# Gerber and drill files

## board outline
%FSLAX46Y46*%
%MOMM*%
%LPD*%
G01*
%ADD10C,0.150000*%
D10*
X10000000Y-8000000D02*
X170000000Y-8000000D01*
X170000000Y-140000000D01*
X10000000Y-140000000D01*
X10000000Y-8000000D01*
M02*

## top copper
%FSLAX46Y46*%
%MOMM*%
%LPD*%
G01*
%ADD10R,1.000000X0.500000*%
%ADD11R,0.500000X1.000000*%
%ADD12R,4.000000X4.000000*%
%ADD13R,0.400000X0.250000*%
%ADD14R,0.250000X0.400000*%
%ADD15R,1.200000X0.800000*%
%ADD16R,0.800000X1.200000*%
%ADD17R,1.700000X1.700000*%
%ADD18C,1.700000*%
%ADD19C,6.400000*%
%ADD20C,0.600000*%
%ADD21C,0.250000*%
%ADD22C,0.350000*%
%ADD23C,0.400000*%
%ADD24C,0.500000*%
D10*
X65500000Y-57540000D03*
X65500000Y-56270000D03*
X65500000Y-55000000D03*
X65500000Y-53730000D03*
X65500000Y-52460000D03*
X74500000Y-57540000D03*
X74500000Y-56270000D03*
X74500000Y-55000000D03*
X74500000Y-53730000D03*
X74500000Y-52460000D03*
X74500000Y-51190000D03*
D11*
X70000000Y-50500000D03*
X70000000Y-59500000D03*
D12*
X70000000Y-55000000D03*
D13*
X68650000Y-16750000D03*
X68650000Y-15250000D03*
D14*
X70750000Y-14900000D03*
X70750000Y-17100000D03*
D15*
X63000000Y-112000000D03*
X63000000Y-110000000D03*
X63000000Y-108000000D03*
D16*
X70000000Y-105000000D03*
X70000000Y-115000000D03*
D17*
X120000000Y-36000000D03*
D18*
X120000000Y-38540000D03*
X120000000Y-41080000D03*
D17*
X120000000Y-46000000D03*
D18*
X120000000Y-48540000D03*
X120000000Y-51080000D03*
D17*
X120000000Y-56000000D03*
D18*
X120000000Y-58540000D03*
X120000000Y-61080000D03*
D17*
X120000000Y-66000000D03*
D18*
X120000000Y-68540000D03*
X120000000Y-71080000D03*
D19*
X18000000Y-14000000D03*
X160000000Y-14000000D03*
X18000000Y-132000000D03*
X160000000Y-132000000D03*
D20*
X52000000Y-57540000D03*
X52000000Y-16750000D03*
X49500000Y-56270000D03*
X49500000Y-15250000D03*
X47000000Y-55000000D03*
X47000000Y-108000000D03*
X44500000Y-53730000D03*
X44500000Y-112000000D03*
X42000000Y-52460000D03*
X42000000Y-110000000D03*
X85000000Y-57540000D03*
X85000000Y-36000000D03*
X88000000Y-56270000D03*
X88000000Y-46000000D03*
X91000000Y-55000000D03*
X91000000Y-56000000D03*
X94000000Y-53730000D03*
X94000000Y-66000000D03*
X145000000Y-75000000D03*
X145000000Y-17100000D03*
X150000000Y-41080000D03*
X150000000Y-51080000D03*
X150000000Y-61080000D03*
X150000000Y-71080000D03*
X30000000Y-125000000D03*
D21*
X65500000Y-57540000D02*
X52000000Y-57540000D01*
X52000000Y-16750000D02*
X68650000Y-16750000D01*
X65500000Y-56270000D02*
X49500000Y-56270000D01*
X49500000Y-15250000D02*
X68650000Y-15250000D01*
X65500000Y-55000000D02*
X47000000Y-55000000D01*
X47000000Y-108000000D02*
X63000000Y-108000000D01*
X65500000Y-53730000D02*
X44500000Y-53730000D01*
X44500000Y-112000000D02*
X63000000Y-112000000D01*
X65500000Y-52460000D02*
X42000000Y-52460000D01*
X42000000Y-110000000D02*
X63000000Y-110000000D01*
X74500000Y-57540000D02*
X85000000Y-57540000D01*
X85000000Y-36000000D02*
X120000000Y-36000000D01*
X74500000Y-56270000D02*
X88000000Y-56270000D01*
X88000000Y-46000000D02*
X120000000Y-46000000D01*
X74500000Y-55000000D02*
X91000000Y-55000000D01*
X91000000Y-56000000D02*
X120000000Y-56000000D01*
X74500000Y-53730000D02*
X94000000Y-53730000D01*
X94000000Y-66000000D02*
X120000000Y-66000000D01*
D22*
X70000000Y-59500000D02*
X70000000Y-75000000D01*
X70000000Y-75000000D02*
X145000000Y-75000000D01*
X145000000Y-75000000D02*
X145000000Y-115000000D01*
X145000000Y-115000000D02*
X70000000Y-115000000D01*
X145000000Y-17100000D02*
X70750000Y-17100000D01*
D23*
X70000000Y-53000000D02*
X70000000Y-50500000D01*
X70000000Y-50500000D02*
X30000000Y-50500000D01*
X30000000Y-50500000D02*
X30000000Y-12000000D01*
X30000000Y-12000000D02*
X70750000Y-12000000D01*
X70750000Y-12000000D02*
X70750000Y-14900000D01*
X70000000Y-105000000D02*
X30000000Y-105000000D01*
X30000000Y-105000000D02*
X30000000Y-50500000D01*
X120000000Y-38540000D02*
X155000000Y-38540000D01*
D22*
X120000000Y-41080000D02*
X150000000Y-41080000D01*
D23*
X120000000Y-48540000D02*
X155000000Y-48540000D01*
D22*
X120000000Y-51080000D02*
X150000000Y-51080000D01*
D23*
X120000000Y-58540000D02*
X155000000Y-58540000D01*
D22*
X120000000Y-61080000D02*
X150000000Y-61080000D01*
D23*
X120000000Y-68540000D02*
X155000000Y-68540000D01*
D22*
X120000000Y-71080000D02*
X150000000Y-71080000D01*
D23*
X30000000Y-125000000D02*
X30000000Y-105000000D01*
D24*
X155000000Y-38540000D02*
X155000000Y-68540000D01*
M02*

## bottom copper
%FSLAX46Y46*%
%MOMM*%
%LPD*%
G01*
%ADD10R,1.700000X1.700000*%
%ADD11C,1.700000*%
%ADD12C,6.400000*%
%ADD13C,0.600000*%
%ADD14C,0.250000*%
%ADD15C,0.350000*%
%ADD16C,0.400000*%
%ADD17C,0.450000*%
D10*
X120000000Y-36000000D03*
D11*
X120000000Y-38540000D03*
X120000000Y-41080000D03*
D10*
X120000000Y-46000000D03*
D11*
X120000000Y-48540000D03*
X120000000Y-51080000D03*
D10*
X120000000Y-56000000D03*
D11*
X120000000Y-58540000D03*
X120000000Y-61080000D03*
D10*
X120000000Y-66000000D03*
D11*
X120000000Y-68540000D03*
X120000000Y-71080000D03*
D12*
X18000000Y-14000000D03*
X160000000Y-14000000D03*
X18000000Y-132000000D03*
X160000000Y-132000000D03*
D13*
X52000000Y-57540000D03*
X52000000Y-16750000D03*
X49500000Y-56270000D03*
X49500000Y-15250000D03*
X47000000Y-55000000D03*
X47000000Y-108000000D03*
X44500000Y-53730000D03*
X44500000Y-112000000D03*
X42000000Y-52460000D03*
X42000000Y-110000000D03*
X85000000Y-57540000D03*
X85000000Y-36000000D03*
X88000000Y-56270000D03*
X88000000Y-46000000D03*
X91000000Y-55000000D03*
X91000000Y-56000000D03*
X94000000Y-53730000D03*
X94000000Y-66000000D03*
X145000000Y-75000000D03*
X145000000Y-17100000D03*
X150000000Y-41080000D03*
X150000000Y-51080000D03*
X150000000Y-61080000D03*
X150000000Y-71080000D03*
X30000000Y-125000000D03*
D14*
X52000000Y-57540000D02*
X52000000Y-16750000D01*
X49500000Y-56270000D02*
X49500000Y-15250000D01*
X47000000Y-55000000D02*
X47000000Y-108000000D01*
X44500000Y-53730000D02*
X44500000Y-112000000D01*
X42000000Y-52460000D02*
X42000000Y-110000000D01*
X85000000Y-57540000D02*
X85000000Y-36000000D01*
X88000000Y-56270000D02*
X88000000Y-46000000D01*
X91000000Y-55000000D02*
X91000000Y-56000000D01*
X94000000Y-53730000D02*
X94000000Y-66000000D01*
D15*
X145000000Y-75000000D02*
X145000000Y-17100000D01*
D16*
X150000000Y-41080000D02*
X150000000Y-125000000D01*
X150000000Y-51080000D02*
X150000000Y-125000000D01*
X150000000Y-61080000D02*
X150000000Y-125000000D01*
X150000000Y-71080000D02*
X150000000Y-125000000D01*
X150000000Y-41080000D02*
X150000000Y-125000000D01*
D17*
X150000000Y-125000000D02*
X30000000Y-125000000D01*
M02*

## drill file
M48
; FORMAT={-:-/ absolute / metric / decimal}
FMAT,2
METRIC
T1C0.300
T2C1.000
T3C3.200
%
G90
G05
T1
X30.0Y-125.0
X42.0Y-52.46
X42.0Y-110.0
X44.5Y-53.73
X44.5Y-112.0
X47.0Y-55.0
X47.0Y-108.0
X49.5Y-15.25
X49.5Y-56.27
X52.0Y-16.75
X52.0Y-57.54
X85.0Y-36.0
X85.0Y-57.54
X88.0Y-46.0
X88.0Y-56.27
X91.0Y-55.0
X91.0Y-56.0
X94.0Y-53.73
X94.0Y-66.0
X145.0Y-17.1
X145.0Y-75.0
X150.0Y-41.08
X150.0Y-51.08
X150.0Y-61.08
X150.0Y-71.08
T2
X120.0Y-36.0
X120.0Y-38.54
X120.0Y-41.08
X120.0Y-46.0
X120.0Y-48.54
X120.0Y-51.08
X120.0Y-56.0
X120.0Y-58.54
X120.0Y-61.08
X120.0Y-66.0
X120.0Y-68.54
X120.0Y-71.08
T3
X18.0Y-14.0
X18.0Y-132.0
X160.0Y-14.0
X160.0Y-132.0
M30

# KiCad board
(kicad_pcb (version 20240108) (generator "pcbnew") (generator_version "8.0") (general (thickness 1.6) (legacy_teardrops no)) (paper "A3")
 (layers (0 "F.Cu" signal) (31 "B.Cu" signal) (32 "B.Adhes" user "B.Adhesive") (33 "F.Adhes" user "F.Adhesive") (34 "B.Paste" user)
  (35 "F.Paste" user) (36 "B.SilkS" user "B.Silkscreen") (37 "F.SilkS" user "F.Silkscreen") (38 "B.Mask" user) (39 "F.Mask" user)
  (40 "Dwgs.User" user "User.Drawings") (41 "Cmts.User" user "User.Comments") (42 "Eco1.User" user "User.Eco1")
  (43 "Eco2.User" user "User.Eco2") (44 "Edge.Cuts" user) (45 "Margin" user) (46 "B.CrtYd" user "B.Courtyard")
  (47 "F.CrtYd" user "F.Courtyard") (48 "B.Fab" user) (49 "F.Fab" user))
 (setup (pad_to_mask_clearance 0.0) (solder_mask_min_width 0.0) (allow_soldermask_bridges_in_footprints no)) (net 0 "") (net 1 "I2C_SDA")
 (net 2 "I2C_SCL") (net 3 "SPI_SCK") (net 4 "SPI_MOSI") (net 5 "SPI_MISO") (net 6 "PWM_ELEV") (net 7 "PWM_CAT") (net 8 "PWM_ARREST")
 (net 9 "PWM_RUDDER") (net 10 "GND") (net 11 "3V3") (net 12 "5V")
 (gr_rect (start 10 8) (end 170 140) (stroke (width 0.15) (type solid)) (fill none) (layer "Edge.Cuts"))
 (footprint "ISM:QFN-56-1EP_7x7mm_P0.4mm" (layer "F.Cu") (at 70 55)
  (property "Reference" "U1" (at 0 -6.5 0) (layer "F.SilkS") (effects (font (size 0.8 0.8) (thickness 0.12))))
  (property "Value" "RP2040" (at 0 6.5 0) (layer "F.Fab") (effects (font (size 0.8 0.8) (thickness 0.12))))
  (pad "1" smd rect (at -4.5 2.54) (size 1.0 0.5) (layers "F.Cu" "F.Paste" "F.Mask") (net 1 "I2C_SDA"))
  (pad "2" smd rect (at -4.5 1.27) (size 1.0 0.5) (layers "F.Cu" "F.Paste" "F.Mask") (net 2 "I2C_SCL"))
  (pad "3" smd rect (at -4.5 0) (size 1.0 0.5) (layers "F.Cu" "F.Paste" "F.Mask") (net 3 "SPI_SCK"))
  (pad "4" smd rect (at -4.5 -1.27) (size 1.0 0.5) (layers "F.Cu" "F.Paste" "F.Mask") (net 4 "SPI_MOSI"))
  (pad "5" smd rect (at -4.5 -2.54) (size 1.0 0.5) (layers "F.Cu" "F.Paste" "F.Mask") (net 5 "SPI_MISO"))
  (pad "6" smd rect (at 4.5 2.54) (size 1.0 0.5) (layers "F.Cu" "F.Paste" "F.Mask") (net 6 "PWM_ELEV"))
  (pad "7" smd rect (at 4.5 1.27) (size 1.0 0.5) (layers "F.Cu" "F.Paste" "F.Mask") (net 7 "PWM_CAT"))
  (pad "8" smd rect (at 4.5 0) (size 1.0 0.5) (layers "F.Cu" "F.Paste" "F.Mask") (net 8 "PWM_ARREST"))
  (pad "9" smd rect (at 4.5 -1.27) (size 1.0 0.5) (layers "F.Cu" "F.Paste" "F.Mask") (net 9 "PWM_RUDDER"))
  (pad "12" smd rect (at 4.5 -2.54) (size 1.0 0.5) (layers "F.Cu" "F.Paste" "F.Mask"))
  (pad "13" smd rect (at 4.5 -3.81) (size 1.0 0.5) (layers "F.Cu" "F.Paste" "F.Mask"))
  (pad "10" smd rect (at 0 -4.5) (size 0.5 1.0) (layers "F.Cu" "F.Paste" "F.Mask") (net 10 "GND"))
  (pad "11" smd rect (at 0 4.5) (size 0.5 1.0) (layers "F.Cu" "F.Paste" "F.Mask") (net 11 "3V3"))
  (pad "EP" smd rect (at 0 0) (size 4 4) (layers "F.Cu" "F.Paste" "F.Mask") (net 10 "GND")))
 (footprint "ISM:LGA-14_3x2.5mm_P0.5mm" (layer "F.Cu") (at 70 16)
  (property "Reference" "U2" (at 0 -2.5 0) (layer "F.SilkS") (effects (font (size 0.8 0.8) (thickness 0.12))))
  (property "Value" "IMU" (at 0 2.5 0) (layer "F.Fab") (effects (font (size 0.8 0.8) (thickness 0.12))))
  (pad "1" smd rect (at -1.35 0.75) (size 0.4 0.25) (layers "F.Cu" "F.Paste" "F.Mask") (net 1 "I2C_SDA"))
  (pad "2" smd rect (at -1.35 -0.75) (size 0.4 0.25) (layers "F.Cu" "F.Paste" "F.Mask") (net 2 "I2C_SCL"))
  (pad "3" smd rect (at 0.75 -1.1) (size 0.25 0.4) (layers "F.Cu" "F.Paste" "F.Mask") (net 10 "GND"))
  (pad "4" smd rect (at 0.75 1.1) (size 0.25 0.4) (layers "F.Cu" "F.Paste" "F.Mask") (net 11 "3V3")))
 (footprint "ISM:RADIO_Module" (layer "F.Cu") (at 70 110)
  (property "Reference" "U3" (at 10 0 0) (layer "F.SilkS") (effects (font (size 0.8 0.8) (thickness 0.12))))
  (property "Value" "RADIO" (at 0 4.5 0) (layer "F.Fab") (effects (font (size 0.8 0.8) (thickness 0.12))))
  (pad "1" smd rect (at -7 2) (size 1.2 0.8) (layers "F.Cu" "F.Paste" "F.Mask") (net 4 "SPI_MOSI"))
  (pad "2" smd rect (at -7 0) (size 1.2 0.8) (layers "F.Cu" "F.Paste" "F.Mask") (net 5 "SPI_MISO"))
  (pad "3" smd rect (at -7 -2) (size 1.2 0.8) (layers "F.Cu" "F.Paste" "F.Mask") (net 3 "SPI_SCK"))
  (pad "4" smd rect (at 0 -5) (size 0.8 1.2) (layers "F.Cu" "F.Paste" "F.Mask") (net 10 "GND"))
  (pad "5" smd rect (at 0 5) (size 0.8 1.2) (layers "F.Cu" "F.Paste" "F.Mask") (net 11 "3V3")))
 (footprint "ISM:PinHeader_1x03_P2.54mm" (layer "F.Cu") (at 120 36)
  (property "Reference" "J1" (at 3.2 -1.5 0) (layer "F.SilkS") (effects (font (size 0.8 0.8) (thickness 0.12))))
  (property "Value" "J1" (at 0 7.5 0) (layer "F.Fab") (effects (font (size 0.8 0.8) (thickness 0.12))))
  (pad "1" thru_hole rect (at 0 0) (size 1.7 1.7) (drill 1.0) (layers "*.Cu" "*.Mask") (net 6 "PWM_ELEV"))
  (pad "2" thru_hole circle (at 0 2.54) (size 1.7 1.7) (drill 1.0) (layers "*.Cu" "*.Mask") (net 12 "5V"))
  (pad "3" thru_hole circle (at 0 5.08) (size 1.7 1.7) (drill 1.0) (layers "*.Cu" "*.Mask") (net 10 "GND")))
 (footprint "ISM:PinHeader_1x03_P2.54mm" (layer "F.Cu") (at 120 46)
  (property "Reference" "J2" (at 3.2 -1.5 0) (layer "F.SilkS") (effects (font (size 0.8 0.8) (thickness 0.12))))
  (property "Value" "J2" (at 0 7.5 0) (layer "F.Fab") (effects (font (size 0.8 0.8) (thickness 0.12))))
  (pad "1" thru_hole rect (at 0 0) (size 1.7 1.7) (drill 1.0) (layers "*.Cu" "*.Mask") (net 7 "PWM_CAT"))
  (pad "2" thru_hole circle (at 0 2.54) (size 1.7 1.7) (drill 1.0) (layers "*.Cu" "*.Mask") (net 12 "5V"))
  (pad "3" thru_hole circle (at 0 5.08) (size 1.7 1.7) (drill 1.0) (layers "*.Cu" "*.Mask") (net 10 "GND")))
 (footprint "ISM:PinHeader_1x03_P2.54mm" (layer "F.Cu") (at 120 56)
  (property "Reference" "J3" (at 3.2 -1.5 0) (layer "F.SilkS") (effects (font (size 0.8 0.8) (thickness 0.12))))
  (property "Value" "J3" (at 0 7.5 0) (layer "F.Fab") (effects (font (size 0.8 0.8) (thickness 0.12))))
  (pad "1" thru_hole rect (at 0 0) (size 1.7 1.7) (drill 1.0) (layers "*.Cu" "*.Mask") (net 8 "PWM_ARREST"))
  (pad "2" thru_hole circle (at 0 2.54) (size 1.7 1.7) (drill 1.0) (layers "*.Cu" "*.Mask") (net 12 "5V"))
  (pad "3" thru_hole circle (at 0 5.08) (size 1.7 1.7) (drill 1.0) (layers "*.Cu" "*.Mask") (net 10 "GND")))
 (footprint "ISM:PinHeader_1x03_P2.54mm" (layer "F.Cu") (at 120 66)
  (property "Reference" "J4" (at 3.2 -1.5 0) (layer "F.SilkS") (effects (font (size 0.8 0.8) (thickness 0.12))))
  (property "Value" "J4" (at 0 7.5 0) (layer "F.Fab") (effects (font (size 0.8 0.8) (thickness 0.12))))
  (pad "1" thru_hole rect (at 0 0) (size 1.7 1.7) (drill 1.0) (layers "*.Cu" "*.Mask") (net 9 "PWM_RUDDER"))
  (pad "2" thru_hole circle (at 0 2.54) (size 1.7 1.7) (drill 1.0) (layers "*.Cu" "*.Mask") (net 12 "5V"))
  (pad "3" thru_hole circle (at 0 5.08) (size 1.7 1.7) (drill 1.0) (layers "*.Cu" "*.Mask") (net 10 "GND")))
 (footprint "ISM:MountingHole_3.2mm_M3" (layer "F.Cu") (at 18 14)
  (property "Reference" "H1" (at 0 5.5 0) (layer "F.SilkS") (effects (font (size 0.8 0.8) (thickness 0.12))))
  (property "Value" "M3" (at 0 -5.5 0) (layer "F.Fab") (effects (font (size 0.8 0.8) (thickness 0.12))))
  (pad "" thru_hole circle (at 0 0) (size 6.4 6.4) (drill 3.2) (layers "*.Cu" "*.Mask")))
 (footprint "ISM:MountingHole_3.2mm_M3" (layer "F.Cu") (at 160 14)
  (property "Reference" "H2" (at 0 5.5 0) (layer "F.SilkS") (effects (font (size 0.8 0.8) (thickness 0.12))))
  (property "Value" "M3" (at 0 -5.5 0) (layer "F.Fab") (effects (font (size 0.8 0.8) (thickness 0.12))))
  (pad "" thru_hole circle (at 0 0) (size 6.4 6.4) (drill 3.2) (layers "*.Cu" "*.Mask")))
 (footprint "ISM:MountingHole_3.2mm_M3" (layer "F.Cu") (at 18 132)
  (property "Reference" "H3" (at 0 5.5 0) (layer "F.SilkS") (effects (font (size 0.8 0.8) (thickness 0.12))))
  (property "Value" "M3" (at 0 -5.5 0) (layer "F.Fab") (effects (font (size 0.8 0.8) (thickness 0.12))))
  (pad "" thru_hole circle (at 0 0) (size 6.4 6.4) (drill 3.2) (layers "*.Cu" "*.Mask")))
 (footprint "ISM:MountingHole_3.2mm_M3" (layer "F.Cu") (at 160 132)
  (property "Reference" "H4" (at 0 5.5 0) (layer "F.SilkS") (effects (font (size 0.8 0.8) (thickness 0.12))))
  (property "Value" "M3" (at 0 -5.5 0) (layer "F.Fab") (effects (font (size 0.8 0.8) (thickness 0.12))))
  (pad "" thru_hole circle (at 0 0) (size 6.4 6.4) (drill 3.2) (layers "*.Cu" "*.Mask")))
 (segment (start 65.5 57.54) (end 52.0 57.54) (width 0.25) (layer "F.Cu") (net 1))
 (segment (start 52.0 57.54) (end 52.0 16.75) (width 0.25) (layer "B.Cu") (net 1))
 (segment (start 52.0 16.75) (end 68.65 16.75) (width 0.25) (layer "F.Cu") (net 1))
 (segment (start 65.5 56.27) (end 49.5 56.27) (width 0.25) (layer "F.Cu") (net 2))
 (segment (start 49.5 56.27) (end 49.5 15.25) (width 0.25) (layer "B.Cu") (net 2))
 (segment (start 49.5 15.25) (end 68.65 15.25) (width 0.25) (layer "F.Cu") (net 2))
 (segment (start 65.5 55) (end 47.0 55) (width 0.25) (layer "F.Cu") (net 3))
 (segment (start 47.0 55) (end 47.0 108) (width 0.25) (layer "B.Cu") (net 3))
 (segment (start 47.0 108) (end 63 108) (width 0.25) (layer "F.Cu") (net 3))
 (segment (start 65.5 53.73) (end 44.5 53.73) (width 0.25) (layer "F.Cu") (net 4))
 (segment (start 44.5 53.73) (end 44.5 112) (width 0.25) (layer "B.Cu") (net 4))
 (segment (start 44.5 112) (end 63 112) (width 0.25) (layer "F.Cu") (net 4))
 (segment (start 65.5 52.46) (end 42.0 52.46) (width 0.25) (layer "F.Cu") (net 5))
 (segment (start 42.0 52.46) (end 42.0 110) (width 0.25) (layer "B.Cu") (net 5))
 (segment (start 42.0 110) (end 63 110) (width 0.25) (layer "F.Cu") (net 5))
 (segment (start 74.5 57.54) (end 85 57.54) (width 0.25) (layer "F.Cu") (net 6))
 (segment (start 85 57.54) (end 85 36) (width 0.25) (layer "B.Cu") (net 6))
 (segment (start 85 36) (end 120 36) (width 0.25) (layer "F.Cu") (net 6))
 (segment (start 74.5 56.27) (end 88 56.27) (width 0.25) (layer "F.Cu") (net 7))
 (segment (start 88 56.27) (end 88 46) (width 0.25) (layer "B.Cu") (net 7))
 (segment (start 88 46) (end 120 46) (width 0.25) (layer "F.Cu") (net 7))
 (segment (start 74.5 55) (end 91 55) (width 0.25) (layer "F.Cu") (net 8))
 (segment (start 91 55) (end 91 56) (width 0.25) (layer "B.Cu") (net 8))
 (segment (start 91 56) (end 120 56) (width 0.25) (layer "F.Cu") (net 8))
 (segment (start 74.5 53.73) (end 94 53.73) (width 0.25) (layer "F.Cu") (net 9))
 (segment (start 94 53.73) (end 94 66) (width 0.25) (layer "B.Cu") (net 9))
 (segment (start 94 66) (end 120 66) (width 0.25) (layer "F.Cu") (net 9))
 (segment (start 70 59.5) (end 70 75) (width 0.35) (layer "F.Cu") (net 11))
 (segment (start 70 75) (end 145 75) (width 0.35) (layer "F.Cu") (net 11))
 (segment (start 145 75) (end 145 115) (width 0.35) (layer "F.Cu") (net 11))
 (segment (start 145 115) (end 70 115) (width 0.35) (layer "F.Cu") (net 11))
 (segment (start 145 75) (end 145 17.1) (width 0.35) (layer "B.Cu") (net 11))
 (segment (start 145 17.1) (end 70.75 17.1) (width 0.35) (layer "F.Cu") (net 11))
 (segment (start 70 53) (end 70 50.5) (width 0.4) (layer "F.Cu") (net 10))
 (segment (start 70 50.5) (end 30 50.5) (width 0.4) (layer "F.Cu") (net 10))
 (segment (start 30 50.5) (end 30 12) (width 0.4) (layer "F.Cu") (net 10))
 (segment (start 30 12) (end 70.75 12) (width 0.4) (layer "F.Cu") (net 10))
 (segment (start 70.75 12) (end 70.75 14.9) (width 0.4) (layer "F.Cu") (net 10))
 (segment (start 70 105) (end 30 105) (width 0.4) (layer "F.Cu") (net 10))
 (segment (start 30 105) (end 30 50.5) (width 0.4) (layer "F.Cu") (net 10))
 (segment (start 120 38.54) (end 155 38.54) (width 0.4) (layer "F.Cu") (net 12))
 (segment (start 120 41.08) (end 150 41.08) (width 0.35) (layer "F.Cu") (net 10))
 (segment (start 150 41.08) (end 150 125) (width 0.4) (layer "B.Cu") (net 10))
 (segment (start 120 48.54) (end 155 48.54) (width 0.4) (layer "F.Cu") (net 12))
 (segment (start 120 51.08) (end 150 51.08) (width 0.35) (layer "F.Cu") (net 10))
 (segment (start 150 51.08) (end 150 125) (width 0.4) (layer "B.Cu") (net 10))
 (segment (start 120 58.54) (end 155 58.54) (width 0.4) (layer "F.Cu") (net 12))
 (segment (start 120 61.08) (end 150 61.08) (width 0.35) (layer "F.Cu") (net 10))
 (segment (start 150 61.08) (end 150 125) (width 0.4) (layer "B.Cu") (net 10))
 (segment (start 120 68.54) (end 155 68.54) (width 0.4) (layer "F.Cu") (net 12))
 (segment (start 120 71.08) (end 150 71.08) (width 0.35) (layer "F.Cu") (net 10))
 (segment (start 150 71.08) (end 150 125) (width 0.4) (layer "B.Cu") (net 10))
 (segment (start 150 41.08) (end 150 125) (width 0.4) (layer "B.Cu") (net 10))
 (segment (start 150 125) (end 30 125) (width 0.45) (layer "B.Cu") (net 10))
 (segment (start 30 125) (end 30 105) (width 0.4) (layer "F.Cu") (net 10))
 (segment (start 155 38.54) (end 155 68.54) (width 0.5) (layer "F.Cu") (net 12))
 (via (at 52.0 57.54) (size 0.6) (drill 0.3) (layers "F.Cu" "B.Cu") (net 1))
 (via (at 52.0 16.75) (size 0.6) (drill 0.3) (layers "F.Cu" "B.Cu") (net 1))
 (via (at 49.5 56.27) (size 0.6) (drill 0.3) (layers "F.Cu" "B.Cu") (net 2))
 (via (at 49.5 15.25) (size 0.6) (drill 0.3) (layers "F.Cu" "B.Cu") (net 2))
 (via (at 47.0 55) (size 0.6) (drill 0.3) (layers "F.Cu" "B.Cu") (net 3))
 (via (at 47.0 108) (size 0.6) (drill 0.3) (layers "F.Cu" "B.Cu") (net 3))
 (via (at 44.5 53.73) (size 0.6) (drill 0.3) (layers "F.Cu" "B.Cu") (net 4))
 (via (at 44.5 112) (size 0.6) (drill 0.3) (layers "F.Cu" "B.Cu") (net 4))
 (via (at 42.0 52.46) (size 0.6) (drill 0.3) (layers "F.Cu" "B.Cu") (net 5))
 (via (at 42.0 110) (size 0.6) (drill 0.3) (layers "F.Cu" "B.Cu") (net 5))
 (via (at 85 57.54) (size 0.6) (drill 0.3) (layers "F.Cu" "B.Cu") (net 6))
 (via (at 85 36) (size 0.6) (drill 0.3) (layers "F.Cu" "B.Cu") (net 6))
 (via (at 88 56.27) (size 0.6) (drill 0.3) (layers "F.Cu" "B.Cu") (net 7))
 (via (at 88 46) (size 0.6) (drill 0.3) (layers "F.Cu" "B.Cu") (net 7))
 (via (at 91 55) (size 0.6) (drill 0.3) (layers "F.Cu" "B.Cu") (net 8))
 (via (at 91 56) (size 0.6) (drill 0.3) (layers "F.Cu" "B.Cu") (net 8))
 (via (at 94 53.73) (size 0.6) (drill 0.3) (layers "F.Cu" "B.Cu") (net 9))
 (via (at 94 66) (size 0.6) (drill 0.3) (layers "F.Cu" "B.Cu") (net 9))
 (via (at 145 75) (size 0.6) (drill 0.3) (layers "F.Cu" "B.Cu") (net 11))
 (via (at 145 17.1) (size 0.6) (drill 0.3) (layers "F.Cu" "B.Cu") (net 11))
 (via (at 150 41.08) (size 0.6) (drill 0.3) (layers "F.Cu" "B.Cu") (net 10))
 (via (at 150 51.08) (size 0.6) (drill 0.3) (layers "F.Cu" "B.Cu") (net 10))
 (via (at 150 61.08) (size 0.6) (drill 0.3) (layers "F.Cu" "B.Cu") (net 10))
 (via (at 150 71.08) (size 0.6) (drill 0.3) (layers "F.Cu" "B.Cu") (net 10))
 (via (at 30 125) (size 0.6) (drill 0.3) (layers "F.Cu" "B.Cu") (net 10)))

